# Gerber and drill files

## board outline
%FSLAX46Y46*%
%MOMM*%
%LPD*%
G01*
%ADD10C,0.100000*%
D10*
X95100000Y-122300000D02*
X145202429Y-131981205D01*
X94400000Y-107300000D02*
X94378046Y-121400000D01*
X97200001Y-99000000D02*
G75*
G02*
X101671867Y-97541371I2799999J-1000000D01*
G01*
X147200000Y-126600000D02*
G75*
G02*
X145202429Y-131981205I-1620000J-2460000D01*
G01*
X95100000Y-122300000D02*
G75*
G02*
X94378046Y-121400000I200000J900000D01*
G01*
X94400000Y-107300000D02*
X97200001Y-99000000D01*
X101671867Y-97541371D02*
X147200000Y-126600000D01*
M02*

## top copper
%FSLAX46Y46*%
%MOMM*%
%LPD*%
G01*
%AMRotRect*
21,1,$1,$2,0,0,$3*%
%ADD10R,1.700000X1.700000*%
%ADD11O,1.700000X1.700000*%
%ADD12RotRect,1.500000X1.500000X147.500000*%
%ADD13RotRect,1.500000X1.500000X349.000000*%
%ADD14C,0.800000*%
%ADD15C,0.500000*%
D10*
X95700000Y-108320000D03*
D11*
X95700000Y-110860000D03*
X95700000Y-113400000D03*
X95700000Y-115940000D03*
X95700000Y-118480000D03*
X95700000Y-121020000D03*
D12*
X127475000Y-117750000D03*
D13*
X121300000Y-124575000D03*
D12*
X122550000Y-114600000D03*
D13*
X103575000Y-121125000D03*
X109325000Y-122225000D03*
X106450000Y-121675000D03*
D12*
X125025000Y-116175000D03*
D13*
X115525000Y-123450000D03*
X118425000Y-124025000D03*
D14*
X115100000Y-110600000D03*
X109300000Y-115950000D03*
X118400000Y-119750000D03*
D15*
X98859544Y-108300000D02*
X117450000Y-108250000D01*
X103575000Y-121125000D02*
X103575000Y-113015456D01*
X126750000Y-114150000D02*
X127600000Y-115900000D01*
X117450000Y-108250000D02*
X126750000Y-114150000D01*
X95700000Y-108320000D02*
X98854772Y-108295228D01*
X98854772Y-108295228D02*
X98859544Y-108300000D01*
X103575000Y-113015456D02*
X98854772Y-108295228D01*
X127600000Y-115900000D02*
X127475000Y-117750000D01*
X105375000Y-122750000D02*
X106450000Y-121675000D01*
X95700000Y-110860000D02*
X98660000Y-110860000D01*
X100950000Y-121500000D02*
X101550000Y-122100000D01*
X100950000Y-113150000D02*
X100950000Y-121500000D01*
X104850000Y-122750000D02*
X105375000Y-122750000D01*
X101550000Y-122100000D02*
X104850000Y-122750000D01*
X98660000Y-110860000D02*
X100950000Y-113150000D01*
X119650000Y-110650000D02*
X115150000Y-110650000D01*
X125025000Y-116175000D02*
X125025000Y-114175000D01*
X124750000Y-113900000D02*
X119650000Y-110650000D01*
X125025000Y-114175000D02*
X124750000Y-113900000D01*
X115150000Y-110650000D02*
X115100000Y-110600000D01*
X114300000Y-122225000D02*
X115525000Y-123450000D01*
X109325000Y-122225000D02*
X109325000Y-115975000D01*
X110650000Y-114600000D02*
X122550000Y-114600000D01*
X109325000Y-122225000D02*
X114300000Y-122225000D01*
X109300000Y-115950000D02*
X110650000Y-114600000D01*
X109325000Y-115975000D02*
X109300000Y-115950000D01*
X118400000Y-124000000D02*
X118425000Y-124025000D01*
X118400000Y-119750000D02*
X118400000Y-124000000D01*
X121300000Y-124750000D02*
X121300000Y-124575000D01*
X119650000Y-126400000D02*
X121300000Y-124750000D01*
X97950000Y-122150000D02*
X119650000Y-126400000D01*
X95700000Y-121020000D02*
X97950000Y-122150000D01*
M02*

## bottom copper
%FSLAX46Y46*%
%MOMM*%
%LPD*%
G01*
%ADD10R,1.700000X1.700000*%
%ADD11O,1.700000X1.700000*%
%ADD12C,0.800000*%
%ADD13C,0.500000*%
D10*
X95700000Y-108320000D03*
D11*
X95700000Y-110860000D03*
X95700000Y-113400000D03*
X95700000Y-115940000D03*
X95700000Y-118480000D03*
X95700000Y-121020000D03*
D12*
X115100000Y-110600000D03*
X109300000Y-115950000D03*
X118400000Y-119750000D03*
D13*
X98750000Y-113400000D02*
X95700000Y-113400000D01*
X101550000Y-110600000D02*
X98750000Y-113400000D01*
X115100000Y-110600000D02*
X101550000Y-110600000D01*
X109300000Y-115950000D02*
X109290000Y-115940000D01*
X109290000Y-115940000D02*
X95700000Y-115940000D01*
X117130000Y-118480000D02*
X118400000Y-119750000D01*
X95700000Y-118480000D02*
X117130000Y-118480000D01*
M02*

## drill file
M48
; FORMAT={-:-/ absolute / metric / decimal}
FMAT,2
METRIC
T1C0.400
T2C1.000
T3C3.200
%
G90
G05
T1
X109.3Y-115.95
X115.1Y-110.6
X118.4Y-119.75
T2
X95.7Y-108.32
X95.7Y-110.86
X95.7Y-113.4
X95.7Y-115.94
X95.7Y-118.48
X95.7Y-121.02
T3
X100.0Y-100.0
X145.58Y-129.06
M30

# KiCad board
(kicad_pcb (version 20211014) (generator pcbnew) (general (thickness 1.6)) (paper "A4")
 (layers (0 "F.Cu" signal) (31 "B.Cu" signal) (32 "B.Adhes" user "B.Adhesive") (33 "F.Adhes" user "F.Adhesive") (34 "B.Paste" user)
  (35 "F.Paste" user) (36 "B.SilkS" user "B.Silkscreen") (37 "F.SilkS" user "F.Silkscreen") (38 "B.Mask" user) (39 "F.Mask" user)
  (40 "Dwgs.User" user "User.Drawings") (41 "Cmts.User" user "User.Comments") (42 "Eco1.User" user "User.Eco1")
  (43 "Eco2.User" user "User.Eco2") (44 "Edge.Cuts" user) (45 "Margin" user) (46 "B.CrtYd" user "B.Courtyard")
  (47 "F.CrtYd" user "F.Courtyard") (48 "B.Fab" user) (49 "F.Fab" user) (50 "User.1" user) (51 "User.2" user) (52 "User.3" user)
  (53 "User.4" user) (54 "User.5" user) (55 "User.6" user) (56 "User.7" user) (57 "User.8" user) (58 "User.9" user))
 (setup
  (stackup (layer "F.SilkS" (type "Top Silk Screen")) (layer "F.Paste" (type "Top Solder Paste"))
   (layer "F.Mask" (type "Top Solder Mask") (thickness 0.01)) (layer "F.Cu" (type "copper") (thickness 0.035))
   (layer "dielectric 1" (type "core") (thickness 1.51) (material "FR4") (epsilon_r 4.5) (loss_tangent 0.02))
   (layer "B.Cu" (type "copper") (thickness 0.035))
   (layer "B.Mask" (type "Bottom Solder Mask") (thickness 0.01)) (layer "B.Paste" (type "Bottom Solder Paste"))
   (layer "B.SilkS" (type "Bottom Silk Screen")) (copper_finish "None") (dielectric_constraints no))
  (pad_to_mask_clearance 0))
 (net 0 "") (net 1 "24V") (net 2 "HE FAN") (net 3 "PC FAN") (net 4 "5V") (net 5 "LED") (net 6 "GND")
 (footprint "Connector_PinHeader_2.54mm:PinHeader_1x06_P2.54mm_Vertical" (layer "F.Cu") (at 95.7 108.32)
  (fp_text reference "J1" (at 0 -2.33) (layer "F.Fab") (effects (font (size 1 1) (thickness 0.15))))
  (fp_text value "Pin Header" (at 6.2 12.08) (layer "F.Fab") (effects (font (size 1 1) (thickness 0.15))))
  (pad "1" thru_hole rect (at 0 0) (size 1.7 1.7) (drill 1) (layers *.Cu *.Mask) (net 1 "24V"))
  (pad "2" thru_hole oval (at 0 2.54) (size 1.7 1.7) (drill 1) (layers *.Cu *.Mask) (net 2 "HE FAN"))
  (pad "3" thru_hole oval (at 0 5.08) (size 1.7 1.7) (drill 1) (layers *.Cu *.Mask) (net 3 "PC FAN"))
  (pad "4" thru_hole oval (at 0 7.62) (size 1.7 1.7) (drill 1) (layers *.Cu *.Mask) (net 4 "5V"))
  (pad "5" thru_hole oval (at 0 10.16) (size 1.7 1.7) (drill 1) (layers *.Cu *.Mask) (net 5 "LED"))
  (pad "6" thru_hole oval (at 0 12.7) (size 1.7 1.7) (drill 1) (layers *.Cu *.Mask) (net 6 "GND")))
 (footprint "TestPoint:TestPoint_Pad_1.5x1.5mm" (layer "F.Cu") (at 127.475 117.75 147.5)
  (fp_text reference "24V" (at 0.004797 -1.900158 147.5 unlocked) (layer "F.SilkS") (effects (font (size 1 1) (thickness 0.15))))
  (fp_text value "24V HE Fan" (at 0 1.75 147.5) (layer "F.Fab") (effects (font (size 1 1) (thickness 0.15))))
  (pad "1" smd rect (at 0 0 147.5) (size 1.5 1.5) (layers "F.Cu" "F.Mask") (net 1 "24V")))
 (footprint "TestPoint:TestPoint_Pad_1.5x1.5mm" (layer "F.Cu") (at 121.3 124.575 -11)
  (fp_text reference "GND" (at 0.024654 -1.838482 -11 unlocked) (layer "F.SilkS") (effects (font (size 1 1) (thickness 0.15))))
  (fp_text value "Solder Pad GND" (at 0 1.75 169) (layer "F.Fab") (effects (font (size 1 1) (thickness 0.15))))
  (pad "1" smd rect (at 0 0 349) (size 1.5 1.5) (layers "F.Cu" "F.Mask") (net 6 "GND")))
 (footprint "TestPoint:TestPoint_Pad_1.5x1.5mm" (layer "F.Cu") (at 122.55 114.6 147.5)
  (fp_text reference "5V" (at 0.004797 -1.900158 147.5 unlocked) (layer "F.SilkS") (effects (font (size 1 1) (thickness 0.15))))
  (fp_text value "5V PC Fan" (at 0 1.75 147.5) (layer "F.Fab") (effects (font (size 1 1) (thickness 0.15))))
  (pad "1" smd rect (at 0 0 147.5) (size 1.5 1.5) (layers "F.Cu" "F.Mask") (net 4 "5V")))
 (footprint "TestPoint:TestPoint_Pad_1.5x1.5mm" (layer "F.Cu") (at 103.575 121.125 -11)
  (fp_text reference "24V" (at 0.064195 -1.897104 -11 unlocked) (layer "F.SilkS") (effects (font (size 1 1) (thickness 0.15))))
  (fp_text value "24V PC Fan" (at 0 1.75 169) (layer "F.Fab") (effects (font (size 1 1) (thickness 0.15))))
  (pad "1" smd rect (at 0 0 349) (size 1.5 1.5) (layers "F.Cu" "F.Mask") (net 1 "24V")))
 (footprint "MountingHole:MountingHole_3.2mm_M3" (layer "F.Cu") (at 145.58 129.06)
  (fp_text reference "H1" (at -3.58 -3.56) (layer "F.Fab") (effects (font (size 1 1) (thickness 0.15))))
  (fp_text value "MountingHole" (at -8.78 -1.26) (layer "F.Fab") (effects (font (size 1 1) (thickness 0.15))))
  (pad "" np_thru_hole circle (at 0 0) (size 3.2 3.2) (drill 3.2) (layers *.Cu *.Mask)))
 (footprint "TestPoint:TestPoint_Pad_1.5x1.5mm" (layer "F.Cu") (at 109.325 122.225 -11)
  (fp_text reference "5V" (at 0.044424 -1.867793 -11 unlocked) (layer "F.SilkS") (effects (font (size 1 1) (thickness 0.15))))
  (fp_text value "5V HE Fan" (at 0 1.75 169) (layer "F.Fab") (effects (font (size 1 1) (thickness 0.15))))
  (pad "1" smd rect (at 0 0 349) (size 1.5 1.5) (layers "F.Cu" "F.Mask") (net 4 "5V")))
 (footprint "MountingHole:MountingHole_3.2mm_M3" (layer "F.Cu") (at 100 100)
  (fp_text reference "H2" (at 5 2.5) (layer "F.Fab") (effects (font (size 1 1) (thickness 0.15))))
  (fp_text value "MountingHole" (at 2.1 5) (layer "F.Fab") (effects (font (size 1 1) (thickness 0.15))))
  (pad "" np_thru_hole circle (at 0 0) (size 3.2 3.2) (drill 3.2) (layers *.Cu *.Mask)))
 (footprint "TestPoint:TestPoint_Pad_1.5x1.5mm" (layer "F.Cu") (at 106.45 121.675 -11)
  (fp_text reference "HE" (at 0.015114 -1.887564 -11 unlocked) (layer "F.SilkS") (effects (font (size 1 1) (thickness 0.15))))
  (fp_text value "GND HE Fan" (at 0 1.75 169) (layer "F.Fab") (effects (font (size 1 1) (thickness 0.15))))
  (pad "1" smd rect (at 0 0 349) (size 1.5 1.5) (layers "F.Cu" "F.Mask") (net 2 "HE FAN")))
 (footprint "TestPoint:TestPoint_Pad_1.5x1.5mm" (layer "F.Cu") (at 125.025 116.175 147.5)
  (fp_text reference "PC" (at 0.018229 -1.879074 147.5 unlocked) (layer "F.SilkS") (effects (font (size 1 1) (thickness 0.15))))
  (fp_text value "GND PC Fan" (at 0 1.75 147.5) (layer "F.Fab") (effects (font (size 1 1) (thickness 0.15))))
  (pad "1" smd rect (at 0 0 147.5) (size 1.5 1.5) (layers "F.Cu" "F.Mask") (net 3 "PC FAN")))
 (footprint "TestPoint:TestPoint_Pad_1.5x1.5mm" (layer "F.Cu") (at 115.525 123.45 -11)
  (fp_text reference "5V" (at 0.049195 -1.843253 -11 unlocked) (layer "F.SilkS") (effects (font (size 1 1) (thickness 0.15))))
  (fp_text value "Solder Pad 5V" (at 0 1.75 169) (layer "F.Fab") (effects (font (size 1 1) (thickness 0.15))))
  (pad "1" smd rect (at 0 0 349) (size 1.5 1.5) (layers "F.Cu" "F.Mask") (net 4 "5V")))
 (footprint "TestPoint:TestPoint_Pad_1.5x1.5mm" (layer "F.Cu") (at 118.425 124.025 -11)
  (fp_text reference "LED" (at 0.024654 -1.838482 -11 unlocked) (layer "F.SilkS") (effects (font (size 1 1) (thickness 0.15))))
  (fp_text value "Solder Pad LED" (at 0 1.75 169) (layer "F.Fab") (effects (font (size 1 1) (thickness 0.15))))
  (pad "1" smd rect (at 0 0 349) (size 1.5 1.5) (layers "F.Cu" "F.Mask") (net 5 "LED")))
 (gr_line (start 95.1 122.3) (end 145.202429 131.981205) (layer "Edge.Cuts") (width 0.1))
 (gr_line (start 94.4 107.3) (end 94.378046 121.4) (layer "Edge.Cuts") (width 0.1))
 (gr_arc (start 97.200001 99) (mid 99.078008 97.173355) (end 101.671867 97.541371) (layer "Edge.Cuts") (width 0.1))
 (gr_arc (start 147.2 126.6) (mid 148.341386 130.085061) (end 145.202429 131.981205) (layer "Edge.Cuts") (width 0.1))
 (gr_arc (start 95.1 122.3) (mid 94.580837 121.976892) (end 94.378046 121.4) (layer "Edge.Cuts") (width 0.1))
 (gr_line (start 94.4 107.3) (end 97.200001 99) (layer "Edge.Cuts") (width 0.1))
 (gr_line (start 101.671867 97.541371) (end 147.2 126.6) (layer "Edge.Cuts") (width 0.1))
 (segment (start 98.859544 108.3) (end 117.45 108.25) (width 0.5) (layer "F.Cu") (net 1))
 (segment (start 103.575 121.125) (end 103.575 113.015456) (width 0.5) (layer "F.Cu") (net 1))
 (segment (start 126.75 114.15) (end 127.6 115.9) (width 0.5) (layer "F.Cu") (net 1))
 (segment (start 117.45 108.25) (end 126.75 114.15) (width 0.5) (layer "F.Cu") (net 1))
 (segment (start 95.7 108.32) (end 98.854772 108.295228) (width 0.5) (layer "F.Cu") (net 1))
 (segment (start 98.854772 108.295228) (end 98.859544 108.3) (width 0.5) (layer "F.Cu") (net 1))
 (segment (start 103.575 113.015456) (end 98.854772 108.295228) (width 0.5) (layer "F.Cu") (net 1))
 (segment (start 127.6 115.9) (end 127.475 117.75) (width 0.5) (layer "F.Cu") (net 1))
 (segment (start 105.375 122.75) (end 106.45 121.675) (width 0.5) (layer "F.Cu") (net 2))
 (segment (start 95.7 110.86) (end 98.66 110.86) (width 0.5) (layer "F.Cu") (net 2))
 (segment (start 100.95 121.5) (end 101.55 122.1) (width 0.5) (layer "F.Cu") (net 2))
 (segment (start 100.95 113.15) (end 100.95 121.5) (width 0.5) (layer "F.Cu") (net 2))
 (segment (start 104.85 122.75) (end 105.375 122.75) (width 0.5) (layer "F.Cu") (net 2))
 (segment (start 101.55 122.1) (end 104.85 122.75) (width 0.5) (layer "F.Cu") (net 2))
 (segment (start 98.66 110.86) (end 100.95 113.15) (width 0.5) (layer "F.Cu") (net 2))
 (segment (start 119.65 110.65) (end 115.15 110.65) (width 0.5) (layer "F.Cu") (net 3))
 (segment (start 125.025 116.175) (end 125.025 114.175) (width 0.5) (layer "F.Cu") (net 3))
 (segment (start 124.75 113.9) (end 119.65 110.65) (width 0.5) (layer "F.Cu") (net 3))
 (segment (start 125.025 114.175) (end 124.75 113.9) (width 0.5) (layer "F.Cu") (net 3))
 (segment (start 115.15 110.65) (end 115.1 110.6) (width 0.5) (layer "F.Cu") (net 3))
 (via (at 115.1 110.6) (size 0.8) (drill 0.4) (layers "F.Cu" "B.Cu") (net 3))
 (segment (start 98.75 113.4) (end 95.7 113.4) (width 0.5) (layer "B.Cu") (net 3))
 (segment (start 101.55 110.6) (end 98.75 113.4) (width 0.5) (layer "B.Cu") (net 3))
 (segment (start 115.1 110.6) (end 101.55 110.6) (width 0.5) (layer "B.Cu") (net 3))
 (segment (start 114.3 122.225) (end 115.525 123.45) (width 0.5) (layer "F.Cu") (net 4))
 (segment (start 109.325 122.225) (end 109.325 115.975) (width 0.5) (layer "F.Cu") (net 4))
 (segment (start 110.65 114.6) (end 122.55 114.6) (width 0.5) (layer "F.Cu") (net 4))
 (segment (start 109.325 122.225) (end 114.3 122.225) (width 0.5) (layer "F.Cu") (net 4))
 (segment (start 109.3 115.95) (end 110.65 114.6) (width 0.5) (layer "F.Cu") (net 4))
 (segment (start 109.325 115.975) (end 109.3 115.95) (width 0.5) (layer "F.Cu") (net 4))
 (via (at 109.3 115.95) (size 0.8) (drill 0.4) (layers "F.Cu" "B.Cu") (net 4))
 (segment (start 109.3 115.95) (end 109.29 115.94) (width 0.5) (layer "B.Cu") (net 4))
 (segment (start 109.29 115.94) (end 95.7 115.94) (width 0.5) (layer "B.Cu") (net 4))
 (segment (start 118.4 124) (end 118.425 124.025) (width 0.5) (layer "F.Cu") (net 5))
 (segment (start 118.4 119.75) (end 118.4 124) (width 0.5) (layer "F.Cu") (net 5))
 (via (at 118.4 119.75) (size 0.8) (drill 0.4) (layers "F.Cu" "B.Cu") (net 5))
 (segment (start 117.13 118.48) (end 118.4 119.75) (width 0.5) (layer "B.Cu") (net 5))
 (segment (start 95.7 118.48) (end 117.13 118.48) (width 0.5) (layer "B.Cu") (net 5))
 (segment (start 121.3 124.75) (end 121.3 124.575) (width 0.5) (layer "F.Cu") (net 6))
 (segment (start 119.65 126.4) (end 121.3 124.75) (width 0.5) (layer "F.Cu") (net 6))
 (segment (start 97.95 122.15) (end 119.65 126.4) (width 0.5) (layer "F.Cu") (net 6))
 (segment (start 95.7 121.02) (end 97.95 122.15) (width 0.5) (layer "F.Cu") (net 6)))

